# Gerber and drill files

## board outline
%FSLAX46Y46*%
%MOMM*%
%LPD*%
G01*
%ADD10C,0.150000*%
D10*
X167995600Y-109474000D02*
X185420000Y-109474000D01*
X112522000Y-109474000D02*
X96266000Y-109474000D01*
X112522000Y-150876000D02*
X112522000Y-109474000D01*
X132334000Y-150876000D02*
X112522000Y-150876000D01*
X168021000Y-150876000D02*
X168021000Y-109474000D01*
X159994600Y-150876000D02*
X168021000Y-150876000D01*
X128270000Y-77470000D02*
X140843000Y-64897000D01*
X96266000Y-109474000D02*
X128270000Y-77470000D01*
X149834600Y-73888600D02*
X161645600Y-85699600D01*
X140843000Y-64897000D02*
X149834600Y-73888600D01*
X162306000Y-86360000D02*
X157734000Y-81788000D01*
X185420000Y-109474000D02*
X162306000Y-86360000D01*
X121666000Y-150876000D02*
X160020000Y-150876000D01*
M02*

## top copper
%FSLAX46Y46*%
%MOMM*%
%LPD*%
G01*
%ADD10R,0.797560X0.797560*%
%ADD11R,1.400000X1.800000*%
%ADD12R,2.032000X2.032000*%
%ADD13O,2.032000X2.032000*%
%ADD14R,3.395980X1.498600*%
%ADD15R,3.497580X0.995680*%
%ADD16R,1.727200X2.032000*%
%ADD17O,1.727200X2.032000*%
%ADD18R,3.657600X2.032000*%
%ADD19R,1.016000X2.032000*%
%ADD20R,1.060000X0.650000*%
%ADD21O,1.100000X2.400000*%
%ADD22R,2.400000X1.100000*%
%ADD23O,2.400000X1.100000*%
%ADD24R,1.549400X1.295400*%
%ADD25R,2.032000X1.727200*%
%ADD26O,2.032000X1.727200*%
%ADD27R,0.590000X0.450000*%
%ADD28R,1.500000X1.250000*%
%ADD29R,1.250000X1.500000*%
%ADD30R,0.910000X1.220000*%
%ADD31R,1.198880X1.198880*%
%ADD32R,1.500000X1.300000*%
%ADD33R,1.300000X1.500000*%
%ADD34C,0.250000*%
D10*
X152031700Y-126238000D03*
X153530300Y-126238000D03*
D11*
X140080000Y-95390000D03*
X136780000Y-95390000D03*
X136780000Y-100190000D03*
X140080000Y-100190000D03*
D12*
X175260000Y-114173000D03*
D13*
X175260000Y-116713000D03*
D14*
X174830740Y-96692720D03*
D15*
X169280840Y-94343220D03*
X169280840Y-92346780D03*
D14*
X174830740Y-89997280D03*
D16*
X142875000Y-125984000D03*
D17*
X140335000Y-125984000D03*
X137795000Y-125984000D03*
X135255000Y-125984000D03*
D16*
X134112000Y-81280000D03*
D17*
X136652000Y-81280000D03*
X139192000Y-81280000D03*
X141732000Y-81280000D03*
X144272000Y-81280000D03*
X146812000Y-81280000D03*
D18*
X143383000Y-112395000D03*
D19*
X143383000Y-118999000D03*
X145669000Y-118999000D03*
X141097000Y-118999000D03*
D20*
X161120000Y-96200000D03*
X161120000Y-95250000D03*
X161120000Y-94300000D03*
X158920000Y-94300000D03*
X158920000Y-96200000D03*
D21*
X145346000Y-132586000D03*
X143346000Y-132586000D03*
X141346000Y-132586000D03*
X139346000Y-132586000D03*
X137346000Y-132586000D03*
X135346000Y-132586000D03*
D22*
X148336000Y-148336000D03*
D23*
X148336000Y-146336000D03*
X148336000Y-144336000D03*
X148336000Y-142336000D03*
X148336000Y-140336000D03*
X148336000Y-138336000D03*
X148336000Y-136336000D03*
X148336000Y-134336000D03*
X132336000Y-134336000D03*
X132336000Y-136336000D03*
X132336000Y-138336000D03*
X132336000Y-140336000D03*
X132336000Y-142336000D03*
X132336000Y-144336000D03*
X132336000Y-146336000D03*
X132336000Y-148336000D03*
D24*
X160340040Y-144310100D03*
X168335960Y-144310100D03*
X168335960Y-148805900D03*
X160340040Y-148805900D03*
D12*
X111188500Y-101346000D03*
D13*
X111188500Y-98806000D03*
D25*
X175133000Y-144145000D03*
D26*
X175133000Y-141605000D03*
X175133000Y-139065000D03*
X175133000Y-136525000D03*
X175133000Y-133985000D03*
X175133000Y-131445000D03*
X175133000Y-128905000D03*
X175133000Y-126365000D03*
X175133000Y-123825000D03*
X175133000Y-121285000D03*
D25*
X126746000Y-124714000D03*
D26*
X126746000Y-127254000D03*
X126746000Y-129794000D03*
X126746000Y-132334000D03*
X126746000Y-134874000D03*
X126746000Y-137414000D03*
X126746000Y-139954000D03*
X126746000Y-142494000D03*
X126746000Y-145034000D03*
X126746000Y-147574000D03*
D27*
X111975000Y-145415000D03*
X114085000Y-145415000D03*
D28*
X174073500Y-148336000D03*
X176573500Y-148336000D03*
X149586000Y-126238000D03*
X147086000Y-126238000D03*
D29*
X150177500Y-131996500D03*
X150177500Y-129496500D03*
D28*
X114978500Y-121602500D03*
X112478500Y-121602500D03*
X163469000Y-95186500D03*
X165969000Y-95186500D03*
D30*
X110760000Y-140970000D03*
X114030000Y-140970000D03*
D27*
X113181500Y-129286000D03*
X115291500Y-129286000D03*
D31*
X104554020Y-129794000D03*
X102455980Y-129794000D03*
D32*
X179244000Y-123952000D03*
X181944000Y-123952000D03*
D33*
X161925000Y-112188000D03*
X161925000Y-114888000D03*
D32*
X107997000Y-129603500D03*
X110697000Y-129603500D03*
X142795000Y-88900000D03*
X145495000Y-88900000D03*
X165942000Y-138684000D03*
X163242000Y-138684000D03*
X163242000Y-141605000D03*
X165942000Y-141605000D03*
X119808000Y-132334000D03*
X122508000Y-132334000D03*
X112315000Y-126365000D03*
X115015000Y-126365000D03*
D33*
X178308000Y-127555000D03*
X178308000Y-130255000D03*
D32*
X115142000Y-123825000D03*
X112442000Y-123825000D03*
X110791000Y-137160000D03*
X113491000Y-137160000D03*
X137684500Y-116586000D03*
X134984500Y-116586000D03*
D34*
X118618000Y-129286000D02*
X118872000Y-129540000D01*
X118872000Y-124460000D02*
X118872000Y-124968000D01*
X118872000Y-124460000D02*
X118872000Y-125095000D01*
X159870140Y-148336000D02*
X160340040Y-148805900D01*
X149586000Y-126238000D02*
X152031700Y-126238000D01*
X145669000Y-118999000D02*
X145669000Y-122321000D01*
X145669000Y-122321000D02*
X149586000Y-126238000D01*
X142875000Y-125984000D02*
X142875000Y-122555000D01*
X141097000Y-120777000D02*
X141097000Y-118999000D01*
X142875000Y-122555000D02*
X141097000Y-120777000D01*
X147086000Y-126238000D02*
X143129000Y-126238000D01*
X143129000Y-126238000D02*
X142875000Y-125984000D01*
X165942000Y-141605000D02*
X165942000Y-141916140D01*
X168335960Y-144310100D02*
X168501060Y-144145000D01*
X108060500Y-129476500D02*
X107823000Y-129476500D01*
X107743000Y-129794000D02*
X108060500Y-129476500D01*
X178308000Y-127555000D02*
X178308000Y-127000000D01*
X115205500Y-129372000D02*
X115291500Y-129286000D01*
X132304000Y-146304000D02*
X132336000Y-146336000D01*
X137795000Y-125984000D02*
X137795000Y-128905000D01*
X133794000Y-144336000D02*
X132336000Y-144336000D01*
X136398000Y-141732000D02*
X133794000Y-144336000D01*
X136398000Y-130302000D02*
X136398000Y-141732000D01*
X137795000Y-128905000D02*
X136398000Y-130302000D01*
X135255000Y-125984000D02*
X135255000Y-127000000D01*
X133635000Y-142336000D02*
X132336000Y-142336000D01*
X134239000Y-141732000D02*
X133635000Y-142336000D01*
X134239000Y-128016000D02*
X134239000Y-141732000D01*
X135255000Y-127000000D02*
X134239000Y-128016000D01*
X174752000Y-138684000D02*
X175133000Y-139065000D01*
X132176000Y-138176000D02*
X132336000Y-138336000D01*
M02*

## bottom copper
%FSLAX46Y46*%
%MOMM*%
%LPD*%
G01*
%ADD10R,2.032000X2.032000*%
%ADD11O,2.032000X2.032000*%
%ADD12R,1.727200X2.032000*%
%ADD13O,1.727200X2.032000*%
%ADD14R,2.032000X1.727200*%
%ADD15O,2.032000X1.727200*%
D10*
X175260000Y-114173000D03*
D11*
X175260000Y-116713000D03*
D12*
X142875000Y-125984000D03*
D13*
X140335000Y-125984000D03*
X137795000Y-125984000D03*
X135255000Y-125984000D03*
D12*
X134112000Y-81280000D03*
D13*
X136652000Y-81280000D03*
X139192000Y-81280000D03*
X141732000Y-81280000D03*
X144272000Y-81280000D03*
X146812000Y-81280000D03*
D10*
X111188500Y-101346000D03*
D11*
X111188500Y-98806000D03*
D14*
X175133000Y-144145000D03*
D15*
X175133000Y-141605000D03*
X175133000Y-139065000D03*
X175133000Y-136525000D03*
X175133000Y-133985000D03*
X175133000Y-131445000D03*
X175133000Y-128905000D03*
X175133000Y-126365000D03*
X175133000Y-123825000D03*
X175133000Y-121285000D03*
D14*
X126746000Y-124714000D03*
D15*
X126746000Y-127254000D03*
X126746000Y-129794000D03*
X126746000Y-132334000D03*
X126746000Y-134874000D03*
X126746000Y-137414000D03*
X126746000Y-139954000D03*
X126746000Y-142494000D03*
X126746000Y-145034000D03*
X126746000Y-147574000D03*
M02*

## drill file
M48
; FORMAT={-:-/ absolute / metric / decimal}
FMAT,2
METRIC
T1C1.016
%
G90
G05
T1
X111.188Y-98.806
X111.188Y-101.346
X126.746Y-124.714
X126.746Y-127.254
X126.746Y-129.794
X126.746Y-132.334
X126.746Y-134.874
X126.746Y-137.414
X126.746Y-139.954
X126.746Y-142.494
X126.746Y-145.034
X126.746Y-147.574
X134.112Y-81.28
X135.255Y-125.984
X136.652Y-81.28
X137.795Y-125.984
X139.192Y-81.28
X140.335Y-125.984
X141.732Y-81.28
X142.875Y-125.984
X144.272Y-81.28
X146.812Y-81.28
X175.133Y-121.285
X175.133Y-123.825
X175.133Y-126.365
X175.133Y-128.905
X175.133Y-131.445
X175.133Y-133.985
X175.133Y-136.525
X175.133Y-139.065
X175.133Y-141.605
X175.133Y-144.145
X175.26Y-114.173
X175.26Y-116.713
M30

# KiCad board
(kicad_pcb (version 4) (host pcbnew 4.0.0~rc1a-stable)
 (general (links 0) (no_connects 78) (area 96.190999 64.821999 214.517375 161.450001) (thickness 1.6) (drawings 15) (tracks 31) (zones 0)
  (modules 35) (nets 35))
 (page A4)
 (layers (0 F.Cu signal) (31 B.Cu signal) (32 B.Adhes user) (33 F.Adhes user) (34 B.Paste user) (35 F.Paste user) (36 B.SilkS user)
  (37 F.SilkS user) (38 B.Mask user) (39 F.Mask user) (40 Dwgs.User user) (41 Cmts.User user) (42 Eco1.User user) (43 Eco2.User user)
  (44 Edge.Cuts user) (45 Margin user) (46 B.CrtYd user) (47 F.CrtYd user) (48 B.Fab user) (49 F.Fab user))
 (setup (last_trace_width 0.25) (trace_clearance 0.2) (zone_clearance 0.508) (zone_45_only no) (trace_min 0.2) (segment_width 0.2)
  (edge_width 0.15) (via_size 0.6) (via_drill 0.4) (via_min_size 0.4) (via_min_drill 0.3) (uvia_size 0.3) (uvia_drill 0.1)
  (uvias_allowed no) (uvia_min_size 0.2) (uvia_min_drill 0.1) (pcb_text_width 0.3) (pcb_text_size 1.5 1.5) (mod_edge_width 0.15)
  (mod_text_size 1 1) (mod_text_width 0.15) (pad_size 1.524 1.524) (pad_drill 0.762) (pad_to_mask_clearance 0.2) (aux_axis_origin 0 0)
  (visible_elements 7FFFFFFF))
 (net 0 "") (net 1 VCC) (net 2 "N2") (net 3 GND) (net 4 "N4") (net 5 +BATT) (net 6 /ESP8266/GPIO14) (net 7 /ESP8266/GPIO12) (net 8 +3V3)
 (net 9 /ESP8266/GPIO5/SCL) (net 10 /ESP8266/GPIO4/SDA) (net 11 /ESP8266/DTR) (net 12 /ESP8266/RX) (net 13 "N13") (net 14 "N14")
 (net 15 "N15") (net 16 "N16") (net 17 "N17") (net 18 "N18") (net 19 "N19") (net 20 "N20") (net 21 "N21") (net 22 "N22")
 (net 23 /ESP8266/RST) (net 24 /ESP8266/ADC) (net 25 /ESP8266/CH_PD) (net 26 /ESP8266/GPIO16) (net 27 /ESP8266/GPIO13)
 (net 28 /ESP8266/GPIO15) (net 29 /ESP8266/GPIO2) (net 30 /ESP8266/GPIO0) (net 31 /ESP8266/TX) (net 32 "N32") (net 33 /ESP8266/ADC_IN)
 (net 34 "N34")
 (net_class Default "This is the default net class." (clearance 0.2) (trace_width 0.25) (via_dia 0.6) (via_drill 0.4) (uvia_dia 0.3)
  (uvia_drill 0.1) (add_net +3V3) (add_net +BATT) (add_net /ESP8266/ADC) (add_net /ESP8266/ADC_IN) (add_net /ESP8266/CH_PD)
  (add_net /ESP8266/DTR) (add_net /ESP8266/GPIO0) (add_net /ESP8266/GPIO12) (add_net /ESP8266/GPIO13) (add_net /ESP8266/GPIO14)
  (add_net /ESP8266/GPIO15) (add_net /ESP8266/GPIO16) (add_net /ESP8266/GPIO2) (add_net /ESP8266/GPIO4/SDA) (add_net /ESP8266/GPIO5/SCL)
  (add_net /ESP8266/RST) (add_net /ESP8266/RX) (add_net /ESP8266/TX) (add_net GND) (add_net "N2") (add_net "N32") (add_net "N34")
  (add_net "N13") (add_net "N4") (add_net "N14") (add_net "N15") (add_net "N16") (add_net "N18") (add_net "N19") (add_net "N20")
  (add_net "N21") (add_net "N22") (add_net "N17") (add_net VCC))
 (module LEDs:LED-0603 (layer F.Cu) (at 152.781 126.238 180)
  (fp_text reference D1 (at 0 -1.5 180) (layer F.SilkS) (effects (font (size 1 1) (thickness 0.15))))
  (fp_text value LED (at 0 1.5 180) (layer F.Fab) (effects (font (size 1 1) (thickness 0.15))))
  (pad 2 smd rect (at 0.7493 0) (size 0.79756 0.79756) (layers F.Cu F.Paste F.Mask) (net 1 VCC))
  (pad 1 smd rect (at -0.7493 0) (size 0.79756 0.79756) (layers F.Cu F.Paste F.Mask) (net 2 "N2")))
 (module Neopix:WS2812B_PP (layer F.Cu) (at 138.43 97.79)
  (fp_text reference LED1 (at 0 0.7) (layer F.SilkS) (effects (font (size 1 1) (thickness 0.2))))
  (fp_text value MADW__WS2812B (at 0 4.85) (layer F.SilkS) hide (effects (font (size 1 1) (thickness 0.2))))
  (pad 3 smd rect (at 1.65 -2.4) (size 1.4 1.8) (layers F.Cu F.Paste F.Mask) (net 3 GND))
  (pad 4 smd rect (at -1.65 -2.4) (size 1.4 1.8) (layers F.Cu F.Paste F.Mask) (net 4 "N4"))
  (pad 1 smd rect (at -1.65 2.4) (size 1.4 1.8) (layers F.Cu F.Paste F.Mask) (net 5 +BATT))
  (pad 2 smd rect (at 1.65 2.4) (size 1.4 1.8) (layers F.Cu F.Paste F.Mask) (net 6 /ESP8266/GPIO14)))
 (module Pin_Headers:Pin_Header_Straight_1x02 (layer F.Cu) (at 175.26 114.173)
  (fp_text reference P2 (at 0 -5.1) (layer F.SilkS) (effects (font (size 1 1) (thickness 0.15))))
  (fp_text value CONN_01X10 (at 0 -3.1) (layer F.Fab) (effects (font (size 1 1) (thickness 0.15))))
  (pad 1 thru_hole rect (at 0 0) (size 2.032 2.032) (drill 1.016) (layers *.Cu *.Mask F.SilkS) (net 5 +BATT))
  (pad 2 thru_hole oval (at 0 2.54) (size 2.032 2.032) (drill 1.016) (layers *.Cu *.Mask F.SilkS) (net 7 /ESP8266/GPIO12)))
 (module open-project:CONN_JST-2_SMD (layer F.Cu) (at 176.53 93.345 90)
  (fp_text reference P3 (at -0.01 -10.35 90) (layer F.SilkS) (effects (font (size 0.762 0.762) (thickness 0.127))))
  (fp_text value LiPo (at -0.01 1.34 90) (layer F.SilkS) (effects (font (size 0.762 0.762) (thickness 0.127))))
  (pad "" smd rect (at -3.34772 -1.69926 90) (size 1.4986 3.39598) (layers F.Cu F.Paste F.Mask))
  (pad 1 smd rect (at -0.99822 -7.24916 90) (size 0.99568 3.49758) (layers F.Cu F.Paste F.Mask) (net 5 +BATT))
  (pad 2 smd rect (at 0.99822 -7.24916 90) (size 0.99568 3.49758) (layers F.Cu F.Paste F.Mask) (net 3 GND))
  (pad "" smd rect (at 3.34772 -1.69926 90) (size 1.4986 3.39598) (layers F.Cu F.Paste F.Mask)))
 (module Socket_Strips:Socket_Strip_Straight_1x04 (layer F.Cu) (at 142.875 125.984 180)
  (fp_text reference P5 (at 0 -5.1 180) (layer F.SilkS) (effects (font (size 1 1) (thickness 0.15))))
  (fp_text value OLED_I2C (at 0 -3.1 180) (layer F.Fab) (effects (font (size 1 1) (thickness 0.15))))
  (pad 1 thru_hole rect (at 0 0 180) (size 1.7272 2.032) (drill 1.016) (layers *.Cu *.Mask F.SilkS) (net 3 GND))
  (pad 2 thru_hole oval (at 2.54 0 180) (size 1.7272 2.032) (drill 1.016) (layers *.Cu *.Mask F.SilkS) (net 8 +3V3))
  (pad 3 thru_hole oval (at 5.08 0 180) (size 1.7272 2.032) (drill 1.016) (layers *.Cu *.Mask F.SilkS) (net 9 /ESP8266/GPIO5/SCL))
  (pad 4 thru_hole oval (at 7.62 0 180) (size 1.7272 2.032) (drill 1.016) (layers *.Cu *.Mask F.SilkS) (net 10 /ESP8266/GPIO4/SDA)))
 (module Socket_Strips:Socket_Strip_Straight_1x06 (layer F.Cu) (at 134.112 81.28)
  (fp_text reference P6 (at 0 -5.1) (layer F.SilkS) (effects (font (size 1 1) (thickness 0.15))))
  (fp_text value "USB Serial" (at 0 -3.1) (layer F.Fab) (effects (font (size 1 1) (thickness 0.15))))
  (pad 1 thru_hole rect (at 0 0) (size 1.7272 2.032) (drill 1.016) (layers *.Cu *.Mask F.SilkS) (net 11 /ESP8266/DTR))
  (pad 2 thru_hole oval (at 2.54 0) (size 1.7272 2.032) (drill 1.016) (layers *.Cu *.Mask F.SilkS) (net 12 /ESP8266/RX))
  (pad 3 thru_hole oval (at 5.08 0) (size 1.7272 2.032) (drill 1.016) (layers *.Cu *.Mask F.SilkS) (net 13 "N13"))
  (pad 4 thru_hole oval (at 7.62 0) (size 1.7272 2.032) (drill 1.016) (layers *.Cu *.Mask F.SilkS) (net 1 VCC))
  (pad 5 thru_hole oval (at 10.16 0) (size 1.7272 2.032) (drill 1.016) (layers *.Cu *.Mask F.SilkS) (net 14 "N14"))
  (pad 6 thru_hole oval (at 12.7 0) (size 1.7272 2.032) (drill 1.016) (layers *.Cu *.Mask F.SilkS) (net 3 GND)))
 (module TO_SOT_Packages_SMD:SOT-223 (layer F.Cu) (at 143.383 115.697)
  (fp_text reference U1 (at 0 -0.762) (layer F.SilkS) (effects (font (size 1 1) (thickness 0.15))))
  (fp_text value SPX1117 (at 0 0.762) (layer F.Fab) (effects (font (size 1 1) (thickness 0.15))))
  (pad 4 smd rect (at 0 -3.302) (size 3.6576 2.032) (layers F.Cu F.Paste F.Mask))
  (pad 2 smd rect (at 0 3.302) (size 1.016 2.032) (layers F.Cu F.Paste F.Mask) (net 8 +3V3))
  (pad 3 smd rect (at 2.286 3.302) (size 1.016 2.032) (layers F.Cu F.Paste F.Mask) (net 1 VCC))
  (pad 1 smd rect (at -2.286 3.302) (size 1.016 2.032) (layers F.Cu F.Paste F.Mask) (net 3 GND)))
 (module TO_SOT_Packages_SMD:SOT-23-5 (layer F.Cu) (at 160.02 95.25 180)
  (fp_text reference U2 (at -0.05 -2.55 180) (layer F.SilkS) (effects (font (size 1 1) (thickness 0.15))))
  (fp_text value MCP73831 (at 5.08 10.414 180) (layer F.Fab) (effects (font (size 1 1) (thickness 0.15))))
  (pad 1 smd rect (at -1.1 -0.95 180) (size 1.06 0.65) (layers F.Cu F.Paste F.Mask) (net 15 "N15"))
  (pad 2 smd rect (at -1.1 0 180) (size 1.06 0.65) (layers F.Cu F.Paste F.Mask) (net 3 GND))
  (pad 3 smd rect (at -1.1 0.95 180) (size 1.06 0.65) (layers F.Cu F.Paste F.Mask) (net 5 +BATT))
  (pad 4 smd rect (at 1.1 0.95 180) (size 1.06 0.65) (layers F.Cu F.Paste F.Mask) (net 1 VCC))
  (pad 5 smd rect (at 1.1 -0.95 180) (size 1.06 0.65) (layers F.Cu F.Paste F.Mask) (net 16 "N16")))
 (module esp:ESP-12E (layer F.Cu) (at 148.336 148.336 180)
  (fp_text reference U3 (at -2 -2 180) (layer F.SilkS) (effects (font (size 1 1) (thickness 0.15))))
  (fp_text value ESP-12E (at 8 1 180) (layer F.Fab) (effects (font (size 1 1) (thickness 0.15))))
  (pad 9 smd oval (at 2.99 15.75 270) (size 2.4 1.1) (layers F.Cu F.Paste F.Mask) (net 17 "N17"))
  (pad 10 smd oval (at 4.99 15.75 270) (size 2.4 1.1) (layers F.Cu F.Paste F.Mask) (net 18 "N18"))
  (pad 11 smd oval (at 6.99 15.75 270) (size 2.4 1.1) (layers F.Cu F.Paste F.Mask) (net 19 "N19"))
  (pad 12 smd oval (at 8.99 15.75 270) (size 2.4 1.1) (layers F.Cu F.Paste F.Mask) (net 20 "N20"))
  (pad 13 smd oval (at 10.99 15.75 270) (size 2.4 1.1) (layers F.Cu F.Paste F.Mask) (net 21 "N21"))
  (pad 14 smd oval (at 12.99 15.75 270) (size 2.4 1.1) (layers F.Cu F.Paste F.Mask) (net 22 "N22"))
  (pad 1 smd rect (at 0 0 180) (size 2.4 1.1) (layers F.Cu F.Paste F.Mask) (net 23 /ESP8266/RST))
  (pad 2 smd oval (at 0 2 180) (size 2.4 1.1) (layers F.Cu F.Paste F.Mask) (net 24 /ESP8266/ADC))
  (pad 3 smd oval (at 0 4 180) (size 2.4 1.1) (layers F.Cu F.Paste F.Mask) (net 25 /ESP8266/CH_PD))
  (pad 4 smd oval (at 0 6 180) (size 2.4 1.1) (layers F.Cu F.Paste F.Mask) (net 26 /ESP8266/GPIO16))
  (pad 5 smd oval (at 0 8 180) (size 2.4 1.1) (layers F.Cu F.Paste F.Mask) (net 6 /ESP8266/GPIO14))
  (pad 6 smd oval (at 0 10 180) (size 2.4 1.1) (layers F.Cu F.Paste F.Mask) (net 7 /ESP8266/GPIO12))
  (pad 7 smd oval (at 0 12 180) (size 2.4 1.1) (layers F.Cu F.Paste F.Mask) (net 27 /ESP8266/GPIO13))
  (pad 8 smd oval (at 0 14 180) (size 2.4 1.1) (layers F.Cu F.Paste F.Mask) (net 8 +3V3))
  (pad 15 smd oval (at 16 14 180) (size 2.4 1.1) (layers F.Cu F.Paste F.Mask) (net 3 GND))
  (pad 16 smd oval (at 16 12 180) (size 2.4 1.1) (layers F.Cu F.Paste F.Mask) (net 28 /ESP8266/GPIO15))
  (pad 17 smd oval (at 16 10 180) (size 2.4 1.1) (layers F.Cu F.Paste F.Mask) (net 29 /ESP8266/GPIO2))
  (pad 18 smd oval (at 16 8 180) (size 2.4 1.1) (layers F.Cu F.Paste F.Mask) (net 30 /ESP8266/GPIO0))
  (pad 19 smd oval (at 16 6 180) (size 2.4 1.1) (layers F.Cu F.Paste F.Mask) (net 10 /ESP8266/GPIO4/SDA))
  (pad 20 smd oval (at 16 4 180) (size 2.4 1.1) (layers F.Cu F.Paste F.Mask) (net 9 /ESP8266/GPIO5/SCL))
  (pad 21 smd oval (at 16 2 180) (size 2.4 1.1) (layers F.Cu F.Paste F.Mask) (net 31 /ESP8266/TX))
  (pad 22 smd oval (at 16 0 180) (size 2.4 1.1) (layers F.Cu F.Paste F.Mask) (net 12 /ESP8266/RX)))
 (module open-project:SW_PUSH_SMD (layer F.Cu) (at 164.338 146.558)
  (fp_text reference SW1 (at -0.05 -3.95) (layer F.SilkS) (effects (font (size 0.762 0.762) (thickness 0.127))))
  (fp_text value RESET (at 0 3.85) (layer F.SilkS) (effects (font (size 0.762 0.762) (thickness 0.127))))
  (pad 1 smd rect (at -3.99796 -2.2479) (size 1.5494 1.2954) (layers F.Cu F.Paste F.Mask) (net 3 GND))
  (pad 1 smd rect (at 3.99796 -2.2479) (size 1.5494 1.2954) (layers F.Cu F.Paste F.Mask) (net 3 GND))
  (pad 2 smd rect (at 3.99796 2.2479) (size 1.5494 1.2954) (layers F.Cu F.Paste F.Mask) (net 23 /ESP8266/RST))
  (pad 2 smd rect (at -3.99796 2.2479) (size 1.5494 1.2954) (layers F.Cu F.Paste F.Mask) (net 23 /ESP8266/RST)))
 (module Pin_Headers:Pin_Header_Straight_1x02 (layer F.Cu) (at 111.1885 101.346 180)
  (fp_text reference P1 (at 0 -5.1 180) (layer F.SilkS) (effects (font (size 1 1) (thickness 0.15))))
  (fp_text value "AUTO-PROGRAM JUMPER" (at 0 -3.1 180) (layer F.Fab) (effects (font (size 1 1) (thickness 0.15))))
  (pad 1 thru_hole rect (at 0 0 180) (size 2.032 2.032) (drill 1.016) (layers *.Cu *.Mask F.SilkS) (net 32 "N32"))
  (pad 2 thru_hole oval (at 0 2.54 180) (size 2.032 2.032) (drill 1.016) (layers *.Cu *.Mask F.SilkS) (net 11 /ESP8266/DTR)))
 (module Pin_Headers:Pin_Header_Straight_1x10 (layer F.Cu) (at 175.133 144.145 180)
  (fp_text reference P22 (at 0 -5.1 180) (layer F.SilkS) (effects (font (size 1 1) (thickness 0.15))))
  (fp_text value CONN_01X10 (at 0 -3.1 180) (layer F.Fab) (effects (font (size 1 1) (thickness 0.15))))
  (pad 1 thru_hole rect (at 0 0 180) (size 2.032 1.7272) (drill 1.016) (layers *.Cu *.Mask F.SilkS) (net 3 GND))
  (pad 2 thru_hole oval (at 0 2.54 180) (size 2.032 1.7272) (drill 1.016) (layers *.Cu *.Mask F.SilkS) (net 30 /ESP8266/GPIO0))
  (pad 3 thru_hole oval (at 0 5.08 180) (size 2.032 1.7272) (drill 1.016) (layers *.Cu *.Mask F.SilkS) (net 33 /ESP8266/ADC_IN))
  (pad 4 thru_hole oval (at 0 7.62 180) (size 2.032 1.7272) (drill 1.016) (layers *.Cu *.Mask F.SilkS) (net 25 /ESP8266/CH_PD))
  (pad 5 thru_hole oval (at 0 10.16 180) (size 2.032 1.7272) (drill 1.016) (layers *.Cu *.Mask F.SilkS) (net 26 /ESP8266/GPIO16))
  (pad 6 thru_hole oval (at 0 12.7 180) (size 2.032 1.7272) (drill 1.016) (layers *.Cu *.Mask F.SilkS) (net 6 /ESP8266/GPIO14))
  (pad 7 thru_hole oval (at 0 15.24 180) (size 2.032 1.7272) (drill 1.016) (layers *.Cu *.Mask F.SilkS) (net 7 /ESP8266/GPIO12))
  (pad 8 thru_hole oval (at 0 17.78 180) (size 2.032 1.7272) (drill 1.016) (layers *.Cu *.Mask F.SilkS) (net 27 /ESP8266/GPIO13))
  (pad 9 thru_hole oval (at 0 20.32 180) (size 2.032 1.7272) (drill 1.016) (layers *.Cu *.Mask F.SilkS) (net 8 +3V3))
  (pad 10 thru_hole oval (at 0 22.86 180) (size 2.032 1.7272) (drill 1.016) (layers *.Cu *.Mask F.SilkS) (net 1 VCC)))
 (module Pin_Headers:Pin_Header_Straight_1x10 (layer F.Cu) (at 126.746 124.714)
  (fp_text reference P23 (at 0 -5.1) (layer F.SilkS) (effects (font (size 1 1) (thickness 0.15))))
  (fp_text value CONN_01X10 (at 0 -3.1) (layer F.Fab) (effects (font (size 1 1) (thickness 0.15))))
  (pad 1 thru_hole rect (at 0 0) (size 2.032 1.7272) (drill 1.016) (layers *.Cu *.Mask F.SilkS) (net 5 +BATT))
  (pad 2 thru_hole oval (at 0 2.54) (size 2.032 1.7272) (drill 1.016) (layers *.Cu *.Mask F.SilkS) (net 28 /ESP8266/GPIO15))
  (pad 3 thru_hole oval (at 0 5.08) (size 2.032 1.7272) (drill 1.016) (layers *.Cu *.Mask F.SilkS) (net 29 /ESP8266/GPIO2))
  (pad 4 thru_hole oval (at 0 7.62) (size 2.032 1.7272) (drill 1.016) (layers *.Cu *.Mask F.SilkS) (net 30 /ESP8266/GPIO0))
  (pad 5 thru_hole oval (at 0 10.16) (size 2.032 1.7272) (drill 1.016) (layers *.Cu *.Mask F.SilkS) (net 3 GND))
  (pad 6 thru_hole oval (at 0 12.7) (size 2.032 1.7272) (drill 1.016) (layers *.Cu *.Mask F.SilkS) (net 10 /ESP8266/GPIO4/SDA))
  (pad 7 thru_hole oval (at 0 15.24) (size 2.032 1.7272) (drill 1.016) (layers *.Cu *.Mask F.SilkS) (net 9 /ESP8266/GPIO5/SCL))
  (pad 8 thru_hole oval (at 0 17.78) (size 2.032 1.7272) (drill 1.016) (layers *.Cu *.Mask F.SilkS) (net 31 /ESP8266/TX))
  (pad 9 thru_hole oval (at 0 20.32) (size 2.032 1.7272) (drill 1.016) (layers *.Cu *.Mask F.SilkS) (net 12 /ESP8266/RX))
  (pad 10 thru_hole oval (at 0 22.86) (size 2.032 1.7272) (drill 1.016) (layers *.Cu *.Mask F.SilkS) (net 3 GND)))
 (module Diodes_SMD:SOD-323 (layer F.Cu) (at 113.03 145.415)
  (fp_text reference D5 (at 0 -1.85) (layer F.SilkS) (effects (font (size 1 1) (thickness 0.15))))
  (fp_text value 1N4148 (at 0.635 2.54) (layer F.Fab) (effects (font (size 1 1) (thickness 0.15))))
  (pad 1 smd rect (at -1.055 0) (size 0.59 0.45) (layers F.Cu F.Paste F.Mask) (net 31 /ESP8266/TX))
  (pad 2 smd rect (at 1.055 0) (size 0.59 0.45) (layers F.Cu F.Paste F.Mask) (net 13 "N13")))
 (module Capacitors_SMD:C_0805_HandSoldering (layer F.Cu) (at 175.3235 148.336)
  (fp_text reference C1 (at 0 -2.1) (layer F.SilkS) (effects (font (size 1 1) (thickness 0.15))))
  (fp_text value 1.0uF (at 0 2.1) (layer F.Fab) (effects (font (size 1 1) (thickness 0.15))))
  (pad 1 smd rect (at -1.25 0) (size 1.5 1.25) (layers F.Cu F.Paste F.Mask) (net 23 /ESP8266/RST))
  (pad 2 smd rect (at 1.25 0) (size 1.5 1.25) (layers F.Cu F.Paste F.Mask) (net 11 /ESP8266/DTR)))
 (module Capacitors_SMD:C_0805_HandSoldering (layer F.Cu) (at 148.336 126.238 180)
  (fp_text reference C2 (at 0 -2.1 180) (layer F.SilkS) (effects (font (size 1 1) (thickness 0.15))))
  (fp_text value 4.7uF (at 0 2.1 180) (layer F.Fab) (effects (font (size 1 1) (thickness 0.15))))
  (pad 1 smd rect (at -1.25 0 180) (size 1.5 1.25) (layers F.Cu F.Paste F.Mask) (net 1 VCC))
  (pad 2 smd rect (at 1.25 0 180) (size 1.5 1.25) (layers F.Cu F.Paste F.Mask) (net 3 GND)))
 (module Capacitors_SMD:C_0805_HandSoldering (layer F.Cu) (at 150.1775 130.7465 90)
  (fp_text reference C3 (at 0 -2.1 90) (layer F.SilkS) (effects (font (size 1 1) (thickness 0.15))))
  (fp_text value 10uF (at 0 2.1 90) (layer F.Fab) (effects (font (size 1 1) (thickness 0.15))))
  (pad 1 smd rect (at -1.25 0 90) (size 1.5 1.25) (layers F.Cu F.Paste F.Mask) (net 8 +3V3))
  (pad 2 smd rect (at 1.25 0 90) (size 1.5 1.25) (layers F.Cu F.Paste F.Mask) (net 3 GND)))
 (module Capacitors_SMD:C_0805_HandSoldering (layer F.Cu) (at 113.7285 121.6025 180)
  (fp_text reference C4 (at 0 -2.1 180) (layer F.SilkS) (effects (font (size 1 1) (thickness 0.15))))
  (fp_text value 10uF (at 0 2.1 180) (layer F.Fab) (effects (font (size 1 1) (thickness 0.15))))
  (pad 1 smd rect (at -1.25 0 180) (size 1.5 1.25) (layers F.Cu F.Paste F.Mask) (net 5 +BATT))
  (pad 2 smd rect (at 1.25 0 180) (size 1.5 1.25) (layers F.Cu F.Paste F.Mask) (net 3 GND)))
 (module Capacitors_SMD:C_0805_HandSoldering (layer F.Cu) (at 164.719 95.1865)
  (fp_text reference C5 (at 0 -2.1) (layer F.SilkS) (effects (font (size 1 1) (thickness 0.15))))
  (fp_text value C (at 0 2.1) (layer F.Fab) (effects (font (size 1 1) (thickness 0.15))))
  (pad 1 smd rect (at -1.25 0) (size 1.5 1.25) (layers F.Cu F.Paste F.Mask) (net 3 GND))
  (pad 2 smd rect (at 1.25 0) (size 1.5 1.25) (layers F.Cu F.Paste F.Mask) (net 5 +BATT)))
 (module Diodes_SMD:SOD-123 (layer F.Cu) (at 112.395 140.97)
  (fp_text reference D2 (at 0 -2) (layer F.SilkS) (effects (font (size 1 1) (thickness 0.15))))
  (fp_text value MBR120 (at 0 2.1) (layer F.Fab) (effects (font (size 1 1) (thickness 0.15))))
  (pad 1 smd rect (at -1.635 0) (size 0.91 1.22) (layers F.Cu F.Paste F.Mask) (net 1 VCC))
  (pad 2 smd rect (at 1.635 0) (size 0.91 1.22) (layers F.Cu F.Paste F.Mask) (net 5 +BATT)))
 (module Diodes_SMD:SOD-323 (layer F.Cu) (at 114.2365 129.286)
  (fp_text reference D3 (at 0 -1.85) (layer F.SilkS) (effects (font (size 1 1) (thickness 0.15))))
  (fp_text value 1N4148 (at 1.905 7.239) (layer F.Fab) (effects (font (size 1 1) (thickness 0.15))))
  (pad 1 smd rect (at -1.055 0) (size 0.59 0.45) (layers F.Cu F.Paste F.Mask) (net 32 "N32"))
  (pad 2 smd rect (at 1.055 0) (size 0.59 0.45) (layers F.Cu F.Paste F.Mask) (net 30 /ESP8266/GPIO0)))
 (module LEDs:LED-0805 (layer F.Cu) (at 103.505 129.794)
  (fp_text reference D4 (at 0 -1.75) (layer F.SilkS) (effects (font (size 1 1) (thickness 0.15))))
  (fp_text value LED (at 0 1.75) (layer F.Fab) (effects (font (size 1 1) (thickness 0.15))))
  (pad 2 smd rect (at 1.04902 0 180) (size 1.19888 1.19888) (layers F.Cu F.Paste F.Mask) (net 8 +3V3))
  (pad 1 smd rect (at -1.04902 0 180) (size 1.19888 1.19888) (layers F.Cu F.Paste F.Mask) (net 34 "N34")))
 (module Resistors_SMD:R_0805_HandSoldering (layer F.Cu) (at 180.594 123.952)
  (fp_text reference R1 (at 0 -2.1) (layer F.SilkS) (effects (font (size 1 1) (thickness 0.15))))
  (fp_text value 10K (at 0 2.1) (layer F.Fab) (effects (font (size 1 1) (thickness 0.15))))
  (pad 1 smd rect (at -1.35 0) (size 1.5 1.3) (layers F.Cu F.Paste F.Mask) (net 8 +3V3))
  (pad 2 smd rect (at 1.35 0) (size 1.5 1.3) (layers F.Cu F.Paste F.Mask) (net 23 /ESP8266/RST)))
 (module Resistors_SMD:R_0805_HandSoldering (layer F.Cu) (at 161.925 113.538 270)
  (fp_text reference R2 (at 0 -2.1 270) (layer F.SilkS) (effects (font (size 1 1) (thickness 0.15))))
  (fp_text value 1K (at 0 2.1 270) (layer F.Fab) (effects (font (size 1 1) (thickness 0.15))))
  (pad 1 smd rect (at -1.35 0 270) (size 1.5 1.3) (layers F.Cu F.Paste F.Mask) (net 15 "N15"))
  (pad 2 smd rect (at 1.35 0 270) (size 1.5 1.3) (layers F.Cu F.Paste F.Mask) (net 2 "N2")))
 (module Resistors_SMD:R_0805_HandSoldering (layer F.Cu) (at 109.347 129.6035)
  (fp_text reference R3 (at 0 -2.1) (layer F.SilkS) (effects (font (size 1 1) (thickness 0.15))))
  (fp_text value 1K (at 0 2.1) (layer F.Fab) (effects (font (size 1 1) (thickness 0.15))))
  (pad 1 smd rect (at -1.35 0) (size 1.5 1.3) (layers F.Cu F.Paste F.Mask) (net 8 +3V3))
  (pad 2 smd rect (at 1.35 0) (size 1.5 1.3) (layers F.Cu F.Paste F.Mask) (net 32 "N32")))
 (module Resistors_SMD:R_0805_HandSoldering (layer F.Cu) (at 144.145 88.9)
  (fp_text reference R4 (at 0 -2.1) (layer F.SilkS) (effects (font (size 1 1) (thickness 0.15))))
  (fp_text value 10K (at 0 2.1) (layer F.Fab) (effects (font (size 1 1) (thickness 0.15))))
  (pad 1 smd rect (at -1.35 0) (size 1.5 1.3) (layers F.Cu F.Paste F.Mask) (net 3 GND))
  (pad 2 smd rect (at 1.35 0) (size 1.5 1.3) (layers F.Cu F.Paste F.Mask) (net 16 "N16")))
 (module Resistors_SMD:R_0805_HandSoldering (layer F.Cu) (at 164.592 138.684 180)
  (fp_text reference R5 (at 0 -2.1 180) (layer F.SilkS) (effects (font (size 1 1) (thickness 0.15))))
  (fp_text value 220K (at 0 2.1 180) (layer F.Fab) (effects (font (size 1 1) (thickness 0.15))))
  (pad 1 smd rect (at -1.35 0 180) (size 1.5 1.3) (layers F.Cu F.Paste F.Mask) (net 33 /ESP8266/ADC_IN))
  (pad 2 smd rect (at 1.35 0 180) (size 1.5 1.3) (layers F.Cu F.Paste F.Mask) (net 24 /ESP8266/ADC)))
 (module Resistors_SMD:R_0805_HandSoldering (layer F.Cu) (at 164.592 141.605)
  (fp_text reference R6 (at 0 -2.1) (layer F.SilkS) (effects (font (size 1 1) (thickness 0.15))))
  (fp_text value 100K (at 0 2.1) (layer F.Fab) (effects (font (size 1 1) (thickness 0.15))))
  (pad 1 smd rect (at -1.35 0) (size 1.5 1.3) (layers F.Cu F.Paste F.Mask) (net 24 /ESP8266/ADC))
  (pad 2 smd rect (at 1.35 0) (size 1.5 1.3) (layers F.Cu F.Paste F.Mask) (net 3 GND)))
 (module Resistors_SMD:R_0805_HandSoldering (layer F.Cu) (at 121.158 132.334)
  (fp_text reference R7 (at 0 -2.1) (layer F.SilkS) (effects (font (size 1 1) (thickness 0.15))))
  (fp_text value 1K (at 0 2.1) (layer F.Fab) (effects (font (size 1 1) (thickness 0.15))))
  (pad 1 smd rect (at -1.35 0) (size 1.5 1.3) (layers F.Cu F.Paste F.Mask) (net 34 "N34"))
  (pad 2 smd rect (at 1.35 0) (size 1.5 1.3) (layers F.Cu F.Paste F.Mask) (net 30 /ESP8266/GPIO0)))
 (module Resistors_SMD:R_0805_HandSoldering (layer F.Cu) (at 113.665 126.365)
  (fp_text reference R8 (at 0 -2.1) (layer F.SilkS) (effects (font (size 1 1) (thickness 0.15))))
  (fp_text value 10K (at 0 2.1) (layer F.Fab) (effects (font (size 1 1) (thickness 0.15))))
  (pad 1 smd rect (at -1.35 0) (size 1.5 1.3) (layers F.Cu F.Paste F.Mask) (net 8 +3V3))
  (pad 2 smd rect (at 1.35 0) (size 1.5 1.3) (layers F.Cu F.Paste F.Mask) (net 29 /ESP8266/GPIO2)))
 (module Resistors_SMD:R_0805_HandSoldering (layer F.Cu) (at 178.308 128.905 270)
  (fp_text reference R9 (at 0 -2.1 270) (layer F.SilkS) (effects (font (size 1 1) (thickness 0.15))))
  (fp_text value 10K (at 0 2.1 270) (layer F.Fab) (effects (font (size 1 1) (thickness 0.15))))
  (pad 1 smd rect (at -1.35 0 270) (size 1.5 1.3) (layers F.Cu F.Paste F.Mask) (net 8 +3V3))
  (pad 2 smd rect (at 1.35 0 270) (size 1.5 1.3) (layers F.Cu F.Paste F.Mask) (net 25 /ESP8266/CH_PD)))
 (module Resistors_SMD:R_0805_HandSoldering (layer F.Cu) (at 113.792 123.825 180)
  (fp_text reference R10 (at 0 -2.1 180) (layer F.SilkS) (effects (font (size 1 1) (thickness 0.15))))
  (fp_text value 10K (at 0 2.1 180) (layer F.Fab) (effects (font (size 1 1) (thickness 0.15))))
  (pad 1 smd rect (at -1.35 0 180) (size 1.5 1.3) (layers F.Cu F.Paste F.Mask) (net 28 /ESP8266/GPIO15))
  (pad 2 smd rect (at 1.35 0 180) (size 1.5 1.3) (layers F.Cu F.Paste F.Mask) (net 3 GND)))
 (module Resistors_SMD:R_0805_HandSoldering (layer F.Cu) (at 112.141 137.16)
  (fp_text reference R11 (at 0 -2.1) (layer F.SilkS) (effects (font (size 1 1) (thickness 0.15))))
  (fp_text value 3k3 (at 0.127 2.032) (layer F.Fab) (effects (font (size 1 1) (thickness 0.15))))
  (pad 1 smd rect (at -1.35 0) (size 1.5 1.3) (layers F.Cu F.Paste F.Mask) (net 8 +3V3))
  (pad 2 smd rect (at 1.35 0) (size 1.5 1.3) (layers F.Cu F.Paste F.Mask) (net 9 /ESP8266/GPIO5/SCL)))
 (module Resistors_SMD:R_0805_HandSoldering (layer F.Cu) (at 136.3345 116.586 180)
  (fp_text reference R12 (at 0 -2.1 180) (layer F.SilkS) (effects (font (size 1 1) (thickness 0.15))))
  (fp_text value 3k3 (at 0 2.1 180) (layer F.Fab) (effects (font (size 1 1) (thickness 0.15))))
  (pad 1 smd rect (at -1.35 0 180) (size 1.5 1.3) (layers F.Cu F.Paste F.Mask) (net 8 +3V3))
  (pad 2 smd rect (at 1.35 0 180) (size 1.5 1.3) (layers F.Cu F.Paste F.Mask) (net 10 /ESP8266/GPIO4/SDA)))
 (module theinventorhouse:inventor (layer F.Cu) (at 140.208 120.015)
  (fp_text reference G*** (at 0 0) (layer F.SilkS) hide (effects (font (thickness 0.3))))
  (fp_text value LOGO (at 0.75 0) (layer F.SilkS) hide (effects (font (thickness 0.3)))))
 (gr_line (start 167.9956 109.474) (end 185.42 109.474) (angle 90) (layer Edge.Cuts) (width 0.15))
 (gr_line (start 112.522 109.474) (end 96.266 109.474) (angle 90) (layer Edge.Cuts) (width 0.15))
 (gr_line (start 112.522 150.876) (end 112.522 109.474) (angle 90) (layer Edge.Cuts) (width 0.15))
 (gr_line (start 132.334 150.876) (end 112.522 150.876) (angle 90) (layer Edge.Cuts) (width 0.15))
 (gr_line (start 168.021 150.876) (end 168.021 109.474) (angle 90) (layer Edge.Cuts) (width 0.15))
 (gr_line (start 159.9946 150.876) (end 168.021 150.876) (angle 90) (layer Edge.Cuts) (width 0.15))
 (gr_line (start 128.27 77.47) (end 140.843 64.897) (angle 90) (layer Edge.Cuts) (width 0.15))
 (gr_line (start 96.266 109.474) (end 128.27 77.47) (angle 90) (layer Edge.Cuts) (width 0.15))
 (gr_line (start 149.8346 73.8886) (end 161.6456 85.6996) (angle 90) (layer Edge.Cuts) (width 0.15))
 (gr_line (start 140.843 64.897) (end 149.8346 73.8886) (angle 90) (layer Edge.Cuts) (width 0.15))
 (gr_line (start 162.306 86.36) (end 157.734 81.788) (angle 90) (layer Edge.Cuts) (width 0.15))
 (gr_line (start 185.42 109.474) (end 162.306 86.36) (angle 90) (layer Edge.Cuts) (width 0.15))
 (gr_line (start 121.666 150.876) (end 160.02 150.876) (angle 90) (layer Edge.Cuts) (width 0.15))
 (segment (start 118.618 129.286) (end 118.872 129.54) (width 0.25) (layer F.Cu) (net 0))
 (segment (start 118.872 124.46) (end 118.872 124.968) (width 0.25) (layer F.Cu) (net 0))
 (segment (start 118.872 124.46) (end 118.872 125.095) (width 0.25) (layer F.Cu) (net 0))
 (segment (start 159.87014 148.336) (end 160.34004 148.8059) (width 0.25) (layer F.Cu) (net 23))
 (segment (start 149.586 126.238) (end 152.0317 126.238) (width 0.25) (layer F.Cu) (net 1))
 (segment (start 145.669 118.999) (end 145.669 122.321) (width 0.25) (layer F.Cu) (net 1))
 (segment (start 145.669 122.321) (end 149.586 126.238) (width 0.25) (layer F.Cu) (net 1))
 (segment (start 142.875 125.984) (end 142.875 122.555) (width 0.25) (layer F.Cu) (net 3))
 (segment (start 141.097 120.777) (end 141.097 118.999) (width 0.25) (layer F.Cu) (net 3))
 (segment (start 142.875 122.555) (end 141.097 120.777) (width 0.25) (layer F.Cu) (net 3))
 (segment (start 147.086 126.238) (end 143.129 126.238) (width 0.25) (layer F.Cu) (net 3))
 (segment (start 143.129 126.238) (end 142.875 125.984) (width 0.25) (layer F.Cu) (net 3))
 (segment (start 165.942 141.605) (end 165.942 141.91614) (width 0.25) (layer F.Cu) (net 3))
 (segment (start 168.33596 144.3101) (end 168.50106 144.145) (width 0.25) (layer F.Cu) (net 3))
 (segment (start 108.0605 129.4765) (end 107.823 129.4765) (width 0.25) (layer F.Cu) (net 8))
 (segment (start 107.743 129.794) (end 108.0605 129.4765) (width 0.25) (layer F.Cu) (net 8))
 (segment (start 178.308 127.555) (end 178.308 127) (width 0.25) (layer F.Cu) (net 8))
 (segment (start 115.2055 129.372) (end 115.2915 129.286) (width 0.25) (layer F.Cu) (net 30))
 (segment (start 132.304 146.304) (end 132.336 146.336) (width 0.25) (layer F.Cu) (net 31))
 (segment (start 137.795 125.984) (end 137.795 128.905) (width 0.25) (layer F.Cu) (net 9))
 (segment (start 133.794 144.336) (end 132.336 144.336) (width 0.25) (layer F.Cu) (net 9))
 (segment (start 136.398 141.732) (end 133.794 144.336) (width 0.25) (layer F.Cu) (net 9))
 (segment (start 136.398 130.302) (end 136.398 141.732) (width 0.25) (layer F.Cu) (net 9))
 (segment (start 137.795 128.905) (end 136.398 130.302) (width 0.25) (layer F.Cu) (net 9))
 (segment (start 135.255 125.984) (end 135.255 127) (width 0.25) (layer F.Cu) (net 10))
 (segment (start 133.635 142.336) (end 132.336 142.336) (width 0.25) (layer F.Cu) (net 10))
 (segment (start 134.239 141.732) (end 133.635 142.336) (width 0.25) (layer F.Cu) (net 10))
 (segment (start 134.239 128.016) (end 134.239 141.732) (width 0.25) (layer F.Cu) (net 10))
 (segment (start 135.255 127) (end 134.239 128.016) (width 0.25) (layer F.Cu) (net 10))
 (segment (start 174.752 138.684) (end 175.133 139.065) (width 0.25) (layer F.Cu) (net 33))
 (segment (start 132.176 138.176) (end 132.336 138.336) (width 0.25) (layer F.Cu) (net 29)))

